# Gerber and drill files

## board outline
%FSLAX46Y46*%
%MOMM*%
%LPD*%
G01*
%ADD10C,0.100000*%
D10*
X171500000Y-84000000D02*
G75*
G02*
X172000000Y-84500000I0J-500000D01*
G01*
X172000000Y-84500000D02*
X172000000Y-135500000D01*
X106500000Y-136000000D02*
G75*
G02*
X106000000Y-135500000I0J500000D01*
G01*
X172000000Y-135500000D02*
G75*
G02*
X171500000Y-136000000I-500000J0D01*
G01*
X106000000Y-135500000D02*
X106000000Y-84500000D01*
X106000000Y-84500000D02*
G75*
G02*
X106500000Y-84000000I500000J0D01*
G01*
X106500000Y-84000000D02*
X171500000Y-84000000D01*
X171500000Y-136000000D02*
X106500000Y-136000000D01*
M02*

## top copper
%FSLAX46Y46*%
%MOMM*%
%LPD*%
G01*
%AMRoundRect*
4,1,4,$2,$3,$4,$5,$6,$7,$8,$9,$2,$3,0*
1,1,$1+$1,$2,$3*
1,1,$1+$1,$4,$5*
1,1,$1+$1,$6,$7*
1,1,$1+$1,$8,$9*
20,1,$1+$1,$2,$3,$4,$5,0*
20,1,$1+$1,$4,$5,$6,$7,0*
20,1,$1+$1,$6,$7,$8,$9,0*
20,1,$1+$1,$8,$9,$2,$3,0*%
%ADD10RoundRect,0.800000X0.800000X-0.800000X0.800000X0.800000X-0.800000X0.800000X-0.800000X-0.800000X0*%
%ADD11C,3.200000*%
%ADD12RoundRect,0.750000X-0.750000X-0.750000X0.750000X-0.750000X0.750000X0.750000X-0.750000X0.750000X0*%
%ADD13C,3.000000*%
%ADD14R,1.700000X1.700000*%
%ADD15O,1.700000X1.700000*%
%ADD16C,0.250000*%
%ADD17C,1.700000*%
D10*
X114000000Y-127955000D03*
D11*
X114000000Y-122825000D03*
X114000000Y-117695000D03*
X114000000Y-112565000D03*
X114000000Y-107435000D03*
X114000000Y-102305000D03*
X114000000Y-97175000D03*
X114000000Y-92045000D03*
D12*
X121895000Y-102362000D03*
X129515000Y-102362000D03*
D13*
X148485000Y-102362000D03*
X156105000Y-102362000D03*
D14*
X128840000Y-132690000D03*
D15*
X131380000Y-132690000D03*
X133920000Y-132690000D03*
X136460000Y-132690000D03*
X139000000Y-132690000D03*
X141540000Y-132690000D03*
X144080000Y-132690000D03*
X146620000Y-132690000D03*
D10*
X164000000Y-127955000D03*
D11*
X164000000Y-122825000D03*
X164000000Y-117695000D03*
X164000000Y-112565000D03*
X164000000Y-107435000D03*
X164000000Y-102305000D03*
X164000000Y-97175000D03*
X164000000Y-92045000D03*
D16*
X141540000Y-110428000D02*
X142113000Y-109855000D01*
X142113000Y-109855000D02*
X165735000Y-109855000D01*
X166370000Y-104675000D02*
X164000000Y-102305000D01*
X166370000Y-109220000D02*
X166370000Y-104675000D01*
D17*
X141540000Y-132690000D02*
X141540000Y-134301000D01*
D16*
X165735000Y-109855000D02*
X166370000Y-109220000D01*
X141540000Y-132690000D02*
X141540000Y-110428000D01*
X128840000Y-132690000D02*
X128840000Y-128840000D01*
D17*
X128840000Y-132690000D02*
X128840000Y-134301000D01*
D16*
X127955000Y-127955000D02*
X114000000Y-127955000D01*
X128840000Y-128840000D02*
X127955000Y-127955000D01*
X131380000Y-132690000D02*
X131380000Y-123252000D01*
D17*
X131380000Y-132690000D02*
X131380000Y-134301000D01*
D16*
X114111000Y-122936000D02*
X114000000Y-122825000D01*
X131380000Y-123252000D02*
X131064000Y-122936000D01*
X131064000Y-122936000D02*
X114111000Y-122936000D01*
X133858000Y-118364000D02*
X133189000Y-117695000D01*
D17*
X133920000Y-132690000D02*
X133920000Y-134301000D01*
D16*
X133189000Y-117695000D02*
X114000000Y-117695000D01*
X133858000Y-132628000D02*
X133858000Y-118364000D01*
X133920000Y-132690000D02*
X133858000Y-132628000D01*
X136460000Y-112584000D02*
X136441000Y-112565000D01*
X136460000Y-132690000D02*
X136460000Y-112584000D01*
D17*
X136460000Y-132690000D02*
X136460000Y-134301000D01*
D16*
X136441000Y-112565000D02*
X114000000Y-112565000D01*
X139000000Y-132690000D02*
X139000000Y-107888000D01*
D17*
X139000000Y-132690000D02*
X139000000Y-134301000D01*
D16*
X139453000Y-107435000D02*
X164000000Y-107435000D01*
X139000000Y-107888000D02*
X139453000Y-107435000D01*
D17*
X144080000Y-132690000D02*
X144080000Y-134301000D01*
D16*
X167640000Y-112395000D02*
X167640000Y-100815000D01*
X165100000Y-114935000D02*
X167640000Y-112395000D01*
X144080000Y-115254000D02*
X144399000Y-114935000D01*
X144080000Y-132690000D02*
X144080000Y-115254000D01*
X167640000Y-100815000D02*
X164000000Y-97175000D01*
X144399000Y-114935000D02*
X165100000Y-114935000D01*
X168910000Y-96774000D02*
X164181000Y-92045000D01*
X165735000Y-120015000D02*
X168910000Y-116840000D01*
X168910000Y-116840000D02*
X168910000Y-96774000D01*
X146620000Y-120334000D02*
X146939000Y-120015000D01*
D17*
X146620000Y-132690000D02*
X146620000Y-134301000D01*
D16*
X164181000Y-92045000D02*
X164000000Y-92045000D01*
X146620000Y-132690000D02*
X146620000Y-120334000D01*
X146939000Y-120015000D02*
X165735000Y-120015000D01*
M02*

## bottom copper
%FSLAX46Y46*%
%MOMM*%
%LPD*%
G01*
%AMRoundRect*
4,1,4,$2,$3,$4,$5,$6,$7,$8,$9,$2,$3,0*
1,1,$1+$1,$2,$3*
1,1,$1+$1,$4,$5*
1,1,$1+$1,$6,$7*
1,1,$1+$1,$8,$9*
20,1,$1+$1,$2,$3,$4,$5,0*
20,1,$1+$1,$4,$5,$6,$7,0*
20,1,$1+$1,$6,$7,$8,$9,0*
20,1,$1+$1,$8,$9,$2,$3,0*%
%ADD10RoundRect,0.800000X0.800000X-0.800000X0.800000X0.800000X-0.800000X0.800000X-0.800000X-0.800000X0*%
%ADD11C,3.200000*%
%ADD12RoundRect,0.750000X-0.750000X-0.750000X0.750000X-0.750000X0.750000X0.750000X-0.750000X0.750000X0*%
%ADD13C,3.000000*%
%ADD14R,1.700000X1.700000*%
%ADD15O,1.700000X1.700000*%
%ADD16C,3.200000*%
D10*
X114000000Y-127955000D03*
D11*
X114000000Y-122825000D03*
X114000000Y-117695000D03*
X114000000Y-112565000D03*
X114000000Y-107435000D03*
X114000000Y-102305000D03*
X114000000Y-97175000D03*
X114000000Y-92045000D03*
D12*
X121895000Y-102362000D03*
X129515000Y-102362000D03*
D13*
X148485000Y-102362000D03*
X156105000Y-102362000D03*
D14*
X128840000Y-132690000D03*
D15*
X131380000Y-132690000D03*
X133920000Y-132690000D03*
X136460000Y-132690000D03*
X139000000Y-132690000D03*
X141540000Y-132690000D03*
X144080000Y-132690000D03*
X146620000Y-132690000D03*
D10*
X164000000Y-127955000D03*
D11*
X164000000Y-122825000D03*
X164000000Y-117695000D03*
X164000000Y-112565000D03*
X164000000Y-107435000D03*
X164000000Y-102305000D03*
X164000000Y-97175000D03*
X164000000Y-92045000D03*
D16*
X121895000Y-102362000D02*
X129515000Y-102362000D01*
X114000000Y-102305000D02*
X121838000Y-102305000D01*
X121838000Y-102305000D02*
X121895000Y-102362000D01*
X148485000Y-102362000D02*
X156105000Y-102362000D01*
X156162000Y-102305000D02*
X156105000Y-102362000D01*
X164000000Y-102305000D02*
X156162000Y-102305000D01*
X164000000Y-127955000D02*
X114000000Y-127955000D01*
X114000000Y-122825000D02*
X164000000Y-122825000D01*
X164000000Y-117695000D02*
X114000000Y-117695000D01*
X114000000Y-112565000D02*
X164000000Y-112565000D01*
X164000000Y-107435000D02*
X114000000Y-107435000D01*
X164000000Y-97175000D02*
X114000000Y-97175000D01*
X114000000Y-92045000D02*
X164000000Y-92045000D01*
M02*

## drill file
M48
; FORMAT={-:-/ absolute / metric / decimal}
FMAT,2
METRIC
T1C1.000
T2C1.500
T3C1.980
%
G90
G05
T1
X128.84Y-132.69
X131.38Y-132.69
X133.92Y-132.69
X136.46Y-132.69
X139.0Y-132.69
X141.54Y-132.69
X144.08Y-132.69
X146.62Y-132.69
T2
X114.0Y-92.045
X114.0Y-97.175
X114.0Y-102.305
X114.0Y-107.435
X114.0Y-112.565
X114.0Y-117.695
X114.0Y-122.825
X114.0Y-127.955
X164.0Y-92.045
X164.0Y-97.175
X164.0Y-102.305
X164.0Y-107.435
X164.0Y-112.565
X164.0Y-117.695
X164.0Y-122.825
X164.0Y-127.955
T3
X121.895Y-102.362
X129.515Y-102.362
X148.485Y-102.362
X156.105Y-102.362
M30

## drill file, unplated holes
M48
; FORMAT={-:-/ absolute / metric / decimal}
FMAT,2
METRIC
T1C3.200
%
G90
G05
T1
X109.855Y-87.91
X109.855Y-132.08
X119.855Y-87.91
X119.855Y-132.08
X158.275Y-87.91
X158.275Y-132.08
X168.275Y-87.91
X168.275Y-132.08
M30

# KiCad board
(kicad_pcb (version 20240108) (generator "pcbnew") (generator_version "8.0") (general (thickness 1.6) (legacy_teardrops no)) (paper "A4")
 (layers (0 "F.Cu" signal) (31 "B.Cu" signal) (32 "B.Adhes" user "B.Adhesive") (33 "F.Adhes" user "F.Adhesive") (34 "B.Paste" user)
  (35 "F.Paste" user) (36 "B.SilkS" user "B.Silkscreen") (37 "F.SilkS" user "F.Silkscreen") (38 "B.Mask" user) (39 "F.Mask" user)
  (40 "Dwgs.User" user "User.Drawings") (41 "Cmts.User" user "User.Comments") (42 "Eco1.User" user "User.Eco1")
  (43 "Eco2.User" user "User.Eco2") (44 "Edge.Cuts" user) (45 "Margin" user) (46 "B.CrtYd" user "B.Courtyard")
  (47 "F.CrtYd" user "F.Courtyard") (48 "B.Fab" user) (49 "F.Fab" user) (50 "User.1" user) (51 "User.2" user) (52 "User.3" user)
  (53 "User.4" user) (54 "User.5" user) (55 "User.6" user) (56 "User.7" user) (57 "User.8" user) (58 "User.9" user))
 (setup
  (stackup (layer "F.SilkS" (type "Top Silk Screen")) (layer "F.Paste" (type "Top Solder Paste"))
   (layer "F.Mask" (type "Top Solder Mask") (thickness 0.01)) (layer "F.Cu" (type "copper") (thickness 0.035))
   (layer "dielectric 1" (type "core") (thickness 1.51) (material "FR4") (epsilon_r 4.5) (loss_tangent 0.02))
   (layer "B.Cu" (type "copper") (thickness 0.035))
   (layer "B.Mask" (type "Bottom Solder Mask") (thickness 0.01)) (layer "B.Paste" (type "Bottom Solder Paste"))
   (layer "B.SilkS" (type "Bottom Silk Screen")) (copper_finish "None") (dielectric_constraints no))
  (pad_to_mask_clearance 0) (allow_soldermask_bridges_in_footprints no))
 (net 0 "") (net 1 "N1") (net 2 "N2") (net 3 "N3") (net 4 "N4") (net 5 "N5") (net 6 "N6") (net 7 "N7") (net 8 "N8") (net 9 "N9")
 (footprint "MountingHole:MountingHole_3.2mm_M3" (layer "F.Cu") (at 109.855 87.91)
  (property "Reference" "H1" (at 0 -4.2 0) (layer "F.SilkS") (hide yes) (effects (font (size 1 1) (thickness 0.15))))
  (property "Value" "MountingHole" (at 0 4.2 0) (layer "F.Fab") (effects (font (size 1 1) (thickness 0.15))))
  (pad "" np_thru_hole circle (at 0 0) (size 3.2 3.2) (drill 3.2) (layers "*.Cu" "*.Mask")))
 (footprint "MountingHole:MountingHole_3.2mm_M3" (layer "F.Cu") (at 168.275 132.08)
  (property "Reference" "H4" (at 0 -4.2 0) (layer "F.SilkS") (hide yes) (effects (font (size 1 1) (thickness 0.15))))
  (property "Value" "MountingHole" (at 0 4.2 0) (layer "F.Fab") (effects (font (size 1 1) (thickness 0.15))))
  (pad "" np_thru_hole circle (at 0 0) (size 3.2 3.2) (drill 3.2) (layers "*.Cu" "*.Mask")))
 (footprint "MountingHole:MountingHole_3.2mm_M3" (layer "F.Cu") (at 158.275 87.91)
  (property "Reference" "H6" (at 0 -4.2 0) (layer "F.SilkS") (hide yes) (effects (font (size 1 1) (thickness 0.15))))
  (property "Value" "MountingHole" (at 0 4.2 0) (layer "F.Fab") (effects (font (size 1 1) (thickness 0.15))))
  (pad "" np_thru_hole circle (at 0 0) (size 3.2 3.2) (drill 3.2) (layers "*.Cu" "*.Mask")))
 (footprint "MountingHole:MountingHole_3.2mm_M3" (layer "F.Cu") (at 158.275 132.08)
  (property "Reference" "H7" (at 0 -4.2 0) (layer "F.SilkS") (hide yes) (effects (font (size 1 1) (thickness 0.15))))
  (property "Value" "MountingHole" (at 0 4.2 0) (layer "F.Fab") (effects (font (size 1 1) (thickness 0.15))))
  (pad "" np_thru_hole circle (at 0 0) (size 3.2 3.2) (drill 3.2) (layers "*.Cu" "*.Mask")))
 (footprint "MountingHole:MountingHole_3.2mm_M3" (layer "F.Cu") (at 119.855 132.08)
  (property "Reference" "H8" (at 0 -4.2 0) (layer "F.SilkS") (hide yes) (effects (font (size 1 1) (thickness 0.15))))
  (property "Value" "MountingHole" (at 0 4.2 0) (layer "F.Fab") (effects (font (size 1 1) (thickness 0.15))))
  (pad "" np_thru_hole circle (at 0 0) (size 3.2 3.2) (drill 3.2) (layers "*.Cu" "*.Mask")))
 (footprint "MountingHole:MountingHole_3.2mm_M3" (layer "F.Cu") (at 119.855 87.91)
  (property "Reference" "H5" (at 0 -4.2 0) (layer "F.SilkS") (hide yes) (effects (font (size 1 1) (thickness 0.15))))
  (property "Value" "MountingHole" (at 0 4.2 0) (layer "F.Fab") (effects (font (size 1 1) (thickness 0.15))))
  (pad "" np_thru_hole circle (at 0 0) (size 3.2 3.2) (drill 3.2) (layers "*.Cu" "*.Mask")))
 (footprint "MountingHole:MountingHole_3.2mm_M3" (layer "F.Cu") (at 109.855 132.08)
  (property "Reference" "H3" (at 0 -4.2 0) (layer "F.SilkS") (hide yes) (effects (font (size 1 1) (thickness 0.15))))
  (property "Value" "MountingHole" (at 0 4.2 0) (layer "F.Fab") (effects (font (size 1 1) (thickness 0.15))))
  (pad "" np_thru_hole circle (at 0 0) (size 3.2 3.2) (drill 3.2) (layers "*.Cu" "*.Mask")))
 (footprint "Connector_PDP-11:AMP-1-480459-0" (layer "F.Cu") (at 114 110 90)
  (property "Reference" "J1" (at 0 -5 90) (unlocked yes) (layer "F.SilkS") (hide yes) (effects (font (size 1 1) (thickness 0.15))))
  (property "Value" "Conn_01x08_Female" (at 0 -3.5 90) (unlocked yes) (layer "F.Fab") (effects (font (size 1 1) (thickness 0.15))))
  (pad "1" thru_hole roundrect (at -17.955 0 90) (size 3.2 3.2) (drill 1.5) (layers "*.Cu" "*.Mask") (remove_unused_layers no)
   (roundrect_rratio 0.25) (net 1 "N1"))
  (pad "2" thru_hole circle (at -12.825 0 90) (size 3.2 3.2) (drill 1.5) (layers "*.Cu" "*.Mask") (remove_unused_layers no) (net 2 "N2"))
  (pad "3" thru_hole circle (at -7.695 0 90) (size 3.2 3.2) (drill 1.5) (layers "*.Cu" "*.Mask") (remove_unused_layers no) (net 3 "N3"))
  (pad "4" thru_hole circle (at -2.565 0 90) (size 3.2 3.2) (drill 1.5) (layers "*.Cu" "*.Mask") (remove_unused_layers no) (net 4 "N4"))
  (pad "5" thru_hole circle (at 2.565 0 90) (size 3.2 3.2) (drill 1.5) (layers "*.Cu" "*.Mask") (remove_unused_layers no) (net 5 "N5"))
  (pad "6" thru_hole circle (at 7.695 0 90) (size 3.2 3.2) (drill 1.5) (layers "*.Cu" "*.Mask") (remove_unused_layers no) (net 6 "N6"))
  (pad "7" thru_hole circle (at 12.825 0 90) (size 3.2 3.2) (drill 1.5) (layers "*.Cu" "*.Mask") (remove_unused_layers no) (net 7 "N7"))
  (pad "8" thru_hole circle (at 17.955 0 90) (size 3.2 3.2) (drill 1.5) (layers "*.Cu" "*.Mask") (remove_unused_layers no) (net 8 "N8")))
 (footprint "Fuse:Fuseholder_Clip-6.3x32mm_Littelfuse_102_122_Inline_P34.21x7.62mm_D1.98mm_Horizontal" (layer "F.Cu") (at 121.895 102.362)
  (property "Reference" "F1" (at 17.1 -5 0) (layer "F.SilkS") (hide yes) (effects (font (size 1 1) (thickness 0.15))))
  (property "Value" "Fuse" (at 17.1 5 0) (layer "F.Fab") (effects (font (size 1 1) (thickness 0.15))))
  (pad "1" thru_hole roundrect (at 0 0) (size 3 3) (drill 1.98) (layers "*.Cu" "*.Mask") (remove_unused_layers no) (roundrect_rratio 0.25)
   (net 6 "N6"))
  (pad "1" thru_hole roundrect (at 7.62 0) (size 3 3) (drill 1.98) (layers "*.Cu" "*.Mask") (remove_unused_layers no)
   (roundrect_rratio 0.25) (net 6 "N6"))
  (pad "2" thru_hole circle (at 26.59 0) (size 3 3) (drill 1.98) (layers "*.Cu" "*.Mask") (remove_unused_layers no) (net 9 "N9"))
  (pad "2" thru_hole circle (at 34.21 0) (size 3 3) (drill 1.98) (layers "*.Cu" "*.Mask") (remove_unused_layers no) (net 9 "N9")))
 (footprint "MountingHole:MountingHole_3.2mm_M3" (layer "F.Cu") (at 168.275 87.91)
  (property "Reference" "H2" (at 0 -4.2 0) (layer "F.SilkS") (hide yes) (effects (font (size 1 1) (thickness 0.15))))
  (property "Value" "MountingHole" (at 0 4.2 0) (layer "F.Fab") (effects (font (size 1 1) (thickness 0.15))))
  (pad "" np_thru_hole circle (at 0 0) (size 3.2 3.2) (drill 3.2) (layers "*.Cu" "*.Mask")))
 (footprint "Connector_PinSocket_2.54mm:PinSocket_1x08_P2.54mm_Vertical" (layer "F.Cu") (at 128.84 132.69 90)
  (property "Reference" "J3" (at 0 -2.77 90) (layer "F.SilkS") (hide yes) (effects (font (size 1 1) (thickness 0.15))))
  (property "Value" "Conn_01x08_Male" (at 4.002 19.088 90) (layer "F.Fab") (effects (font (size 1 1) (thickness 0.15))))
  (pad "1" thru_hole rect (at 0 0 90) (size 1.7 1.7) (drill 1) (layers "*.Cu" "*.Mask") (remove_unused_layers no) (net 1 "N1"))
  (pad "2" thru_hole oval (at 0 2.54 90) (size 1.7 1.7) (drill 1) (layers "*.Cu" "*.Mask") (remove_unused_layers no) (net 2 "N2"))
  (pad "3" thru_hole oval (at 0 5.08 90) (size 1.7 1.7) (drill 1) (layers "*.Cu" "*.Mask") (remove_unused_layers no) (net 3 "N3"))
  (pad "4" thru_hole oval (at 0 7.62 90) (size 1.7 1.7) (drill 1) (layers "*.Cu" "*.Mask") (remove_unused_layers no) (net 4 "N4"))
  (pad "5" thru_hole oval (at 0 10.16 90) (size 1.7 1.7) (drill 1) (layers "*.Cu" "*.Mask") (remove_unused_layers no) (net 5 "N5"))
  (pad "6" thru_hole oval (at 0 12.7 90) (size 1.7 1.7) (drill 1) (layers "*.Cu" "*.Mask") (remove_unused_layers no) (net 9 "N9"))
  (pad "7" thru_hole oval (at 0 15.24 90) (size 1.7 1.7) (drill 1) (layers "*.Cu" "*.Mask") (remove_unused_layers no) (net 7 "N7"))
  (pad "8" thru_hole oval (at 0 17.78 90) (size 1.7 1.7) (drill 1) (layers "*.Cu" "*.Mask") (remove_unused_layers no) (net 8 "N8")))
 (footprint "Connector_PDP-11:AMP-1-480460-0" (layer "B.Cu") (at 164 110 90)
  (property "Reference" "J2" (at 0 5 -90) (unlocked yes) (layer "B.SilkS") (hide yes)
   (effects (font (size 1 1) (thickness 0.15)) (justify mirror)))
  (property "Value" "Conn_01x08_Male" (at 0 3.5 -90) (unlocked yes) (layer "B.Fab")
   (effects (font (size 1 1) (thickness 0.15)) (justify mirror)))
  (pad "1" thru_hole roundrect (at -17.955 0 90) (size 3.2 3.2) (drill 1.5) (layers "*.Cu" "*.Mask") (remove_unused_layers no)
   (roundrect_rratio 0.25) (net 1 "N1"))
  (pad "2" thru_hole circle (at -12.825 0 90) (size 3.2 3.2) (drill 1.5) (layers "*.Cu" "*.Mask") (remove_unused_layers no) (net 2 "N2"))
  (pad "3" thru_hole circle (at -7.695 0 90) (size 3.2 3.2) (drill 1.5) (layers "*.Cu" "*.Mask") (remove_unused_layers no) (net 3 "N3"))
  (pad "4" thru_hole circle (at -2.565 0 90) (size 3.2 3.2) (drill 1.5) (layers "*.Cu" "*.Mask") (remove_unused_layers no) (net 4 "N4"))
  (pad "5" thru_hole circle (at 2.565 0 90) (size 3.2 3.2) (drill 1.5) (layers "*.Cu" "*.Mask") (remove_unused_layers no) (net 5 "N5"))
  (pad "6" thru_hole circle (at 7.695 0 90) (size 3.2 3.2) (drill 1.5) (layers "*.Cu" "*.Mask") (remove_unused_layers no) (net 9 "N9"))
  (pad "7" thru_hole circle (at 12.825 0 90) (size 3.2 3.2) (drill 1.5) (layers "*.Cu" "*.Mask") (remove_unused_layers no) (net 7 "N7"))
  (pad "8" thru_hole circle (at 17.955 0 90) (size 3.2 3.2) (drill 1.5) (layers "*.Cu" "*.Mask") (remove_unused_layers no) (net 8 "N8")))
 (gr_arc (start 171.5 84) (mid 171.853553 84.146447) (end 172 84.5) (stroke (width 0.1) (type solid)) (layer "Edge.Cuts"))
 (gr_line (start 172 84.5) (end 172 135.5) (stroke (width 0.1) (type solid)) (layer "Edge.Cuts"))
 (gr_arc (start 106.5 136) (mid 106.146447 135.853553) (end 106 135.5) (stroke (width 0.1) (type solid)) (layer "Edge.Cuts"))
 (gr_arc (start 172 135.5) (mid 171.853553 135.853553) (end 171.5 136) (stroke (width 0.1) (type solid)) (layer "Edge.Cuts"))
 (gr_line (start 106 135.5) (end 106 84.5) (stroke (width 0.1) (type solid)) (layer "Edge.Cuts"))
 (gr_arc (start 106 84.5) (mid 106.146447 84.146447) (end 106.5 84) (stroke (width 0.1) (type solid)) (layer "Edge.Cuts"))
 (gr_line (start 106.5 84) (end 171.5 84) (stroke (width 0.1) (type solid)) (layer "Edge.Cuts"))
 (gr_line (start 171.5 136) (end 106.5 136) (stroke (width 0.1) (type solid)) (layer "Edge.Cuts"))
 (segment (start 121.895 102.362) (end 129.515 102.362) (width 3.2) (layer "B.Cu") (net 6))
 (segment (start 114 102.305) (end 121.838 102.305) (width 3.2) (layer "B.Cu") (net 6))
 (segment (start 121.838 102.305) (end 121.895 102.362) (width 3.2) (layer "B.Cu") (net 6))
 (segment (start 141.54 110.428) (end 142.113 109.855) (width 0.25) (layer "F.Cu") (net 9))
 (segment (start 142.113 109.855) (end 165.735 109.855) (width 0.25) (layer "F.Cu") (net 9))
 (segment (start 166.37 104.675) (end 164 102.305) (width 0.25) (layer "F.Cu") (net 9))
 (segment (start 166.37 109.22) (end 166.37 104.675) (width 0.25) (layer "F.Cu") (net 9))
 (segment (start 141.54 132.69) (end 141.54 134.301) (width 1.7) (layer "F.Cu") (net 9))
 (segment (start 165.735 109.855) (end 166.37 109.22) (width 0.25) (layer "F.Cu") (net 9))
 (segment (start 141.54 132.69) (end 141.54 110.428) (width 0.25) (layer "F.Cu") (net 9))
 (segment (start 148.485 102.362) (end 156.105 102.362) (width 3.2) (layer "B.Cu") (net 9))
 (segment (start 156.162 102.305) (end 156.105 102.362) (width 3.2) (layer "B.Cu") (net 9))
 (segment (start 164 102.305) (end 156.162 102.305) (width 3.2) (layer "B.Cu") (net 9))
 (segment (start 128.84 132.69) (end 128.84 128.84) (width 0.25) (layer "F.Cu") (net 1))
 (segment (start 128.84 132.69) (end 128.84 134.301) (width 1.7) (layer "F.Cu") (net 1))
 (segment (start 127.955 127.955) (end 114 127.955) (width 0.25) (layer "F.Cu") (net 1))
 (segment (start 128.84 128.84) (end 127.955 127.955) (width 0.25) (layer "F.Cu") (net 1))
 (segment (start 164 127.955) (end 114 127.955) (width 3.2) (layer "B.Cu") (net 1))
 (segment (start 131.38 132.69) (end 131.38 123.252) (width 0.25) (layer "F.Cu") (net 2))
 (segment (start 131.38 132.69) (end 131.38 134.301) (width 1.7) (layer "F.Cu") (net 2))
 (segment (start 114.111 122.936) (end 114 122.825) (width 0.25) (layer "F.Cu") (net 2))
 (segment (start 131.38 123.252) (end 131.064 122.936) (width 0.25) (layer "F.Cu") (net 2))
 (segment (start 131.064 122.936) (end 114.111 122.936) (width 0.25) (layer "F.Cu") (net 2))
 (segment (start 114 122.825) (end 164 122.825) (width 3.2) (layer "B.Cu") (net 2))
 (segment (start 133.858 118.364) (end 133.189 117.695) (width 0.25) (layer "F.Cu") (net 3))
 (segment (start 133.92 132.69) (end 133.92 134.301) (width 1.7) (layer "F.Cu") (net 3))
 (segment (start 133.189 117.695) (end 114 117.695) (width 0.25) (layer "F.Cu") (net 3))
 (segment (start 133.858 132.628) (end 133.858 118.364) (width 0.25) (layer "F.Cu") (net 3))
 (segment (start 133.92 132.69) (end 133.858 132.628) (width 0.25) (layer "F.Cu") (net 3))
 (segment (start 164 117.695) (end 114 117.695) (width 3.2) (layer "B.Cu") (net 3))
 (segment (start 136.46 112.584) (end 136.441 112.565) (width 0.25) (layer "F.Cu") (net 4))
 (segment (start 136.46 132.69) (end 136.46 112.584) (width 0.25) (layer "F.Cu") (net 4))
 (segment (start 136.46 132.69) (end 136.46 134.301) (width 1.7) (layer "F.Cu") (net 4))
 (segment (start 136.441 112.565) (end 114 112.565) (width 0.25) (layer "F.Cu") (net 4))
 (segment (start 114 112.565) (end 164 112.565) (width 3.2) (layer "B.Cu") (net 4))
 (segment (start 139 132.69) (end 139 107.888) (width 0.25) (layer "F.Cu") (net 5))
 (segment (start 139 132.69) (end 139 134.301) (width 1.7) (layer "F.Cu") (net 5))
 (segment (start 139.453 107.435) (end 164 107.435) (width 0.25) (layer "F.Cu") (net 5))
 (segment (start 139 107.888) (end 139.453 107.435) (width 0.25) (layer "F.Cu") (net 5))
 (segment (start 164 107.435) (end 114 107.435) (width 3.2) (layer "B.Cu") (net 5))
 (segment (start 144.08 132.69) (end 144.08 134.301) (width 1.7) (layer "F.Cu") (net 7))
 (segment (start 167.64 112.395) (end 167.64 100.815) (width 0.25) (layer "F.Cu") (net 7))
 (segment (start 165.1 114.935) (end 167.64 112.395) (width 0.25) (layer "F.Cu") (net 7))
 (segment (start 144.08 115.254) (end 144.399 114.935) (width 0.25) (layer "F.Cu") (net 7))
 (segment (start 144.08 132.69) (end 144.08 115.254) (width 0.25) (layer "F.Cu") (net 7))
 (segment (start 167.64 100.815) (end 164 97.175) (width 0.25) (layer "F.Cu") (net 7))
 (segment (start 144.399 114.935) (end 165.1 114.935) (width 0.25) (layer "F.Cu") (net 7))
 (segment (start 164 97.175) (end 114 97.175) (width 3.2) (layer "B.Cu") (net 7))
 (segment (start 168.91 96.774) (end 164.181 92.045) (width 0.25) (layer "F.Cu") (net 8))
 (segment (start 165.735 120.015) (end 168.91 116.84) (width 0.25) (layer "F.Cu") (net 8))
 (segment (start 168.91 116.84) (end 168.91 96.774) (width 0.25) (layer "F.Cu") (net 8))
 (segment (start 146.62 120.334) (end 146.939 120.015) (width 0.25) (layer "F.Cu") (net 8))
 (segment (start 146.62 132.69) (end 146.62 134.301) (width 1.7) (layer "F.Cu") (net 8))
 (segment (start 164.181 92.045) (end 164 92.045) (width 0.25) (layer "F.Cu") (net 8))
 (segment (start 146.62 132.69) (end 146.62 120.334) (width 0.25) (layer "F.Cu") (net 8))
 (segment (start 146.939 120.015) (end 165.735 120.015) (width 0.25) (layer "F.Cu") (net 8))
 (segment (start 114 92.045) (end 164 92.045) (width 3.2) (layer "B.Cu") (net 8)))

